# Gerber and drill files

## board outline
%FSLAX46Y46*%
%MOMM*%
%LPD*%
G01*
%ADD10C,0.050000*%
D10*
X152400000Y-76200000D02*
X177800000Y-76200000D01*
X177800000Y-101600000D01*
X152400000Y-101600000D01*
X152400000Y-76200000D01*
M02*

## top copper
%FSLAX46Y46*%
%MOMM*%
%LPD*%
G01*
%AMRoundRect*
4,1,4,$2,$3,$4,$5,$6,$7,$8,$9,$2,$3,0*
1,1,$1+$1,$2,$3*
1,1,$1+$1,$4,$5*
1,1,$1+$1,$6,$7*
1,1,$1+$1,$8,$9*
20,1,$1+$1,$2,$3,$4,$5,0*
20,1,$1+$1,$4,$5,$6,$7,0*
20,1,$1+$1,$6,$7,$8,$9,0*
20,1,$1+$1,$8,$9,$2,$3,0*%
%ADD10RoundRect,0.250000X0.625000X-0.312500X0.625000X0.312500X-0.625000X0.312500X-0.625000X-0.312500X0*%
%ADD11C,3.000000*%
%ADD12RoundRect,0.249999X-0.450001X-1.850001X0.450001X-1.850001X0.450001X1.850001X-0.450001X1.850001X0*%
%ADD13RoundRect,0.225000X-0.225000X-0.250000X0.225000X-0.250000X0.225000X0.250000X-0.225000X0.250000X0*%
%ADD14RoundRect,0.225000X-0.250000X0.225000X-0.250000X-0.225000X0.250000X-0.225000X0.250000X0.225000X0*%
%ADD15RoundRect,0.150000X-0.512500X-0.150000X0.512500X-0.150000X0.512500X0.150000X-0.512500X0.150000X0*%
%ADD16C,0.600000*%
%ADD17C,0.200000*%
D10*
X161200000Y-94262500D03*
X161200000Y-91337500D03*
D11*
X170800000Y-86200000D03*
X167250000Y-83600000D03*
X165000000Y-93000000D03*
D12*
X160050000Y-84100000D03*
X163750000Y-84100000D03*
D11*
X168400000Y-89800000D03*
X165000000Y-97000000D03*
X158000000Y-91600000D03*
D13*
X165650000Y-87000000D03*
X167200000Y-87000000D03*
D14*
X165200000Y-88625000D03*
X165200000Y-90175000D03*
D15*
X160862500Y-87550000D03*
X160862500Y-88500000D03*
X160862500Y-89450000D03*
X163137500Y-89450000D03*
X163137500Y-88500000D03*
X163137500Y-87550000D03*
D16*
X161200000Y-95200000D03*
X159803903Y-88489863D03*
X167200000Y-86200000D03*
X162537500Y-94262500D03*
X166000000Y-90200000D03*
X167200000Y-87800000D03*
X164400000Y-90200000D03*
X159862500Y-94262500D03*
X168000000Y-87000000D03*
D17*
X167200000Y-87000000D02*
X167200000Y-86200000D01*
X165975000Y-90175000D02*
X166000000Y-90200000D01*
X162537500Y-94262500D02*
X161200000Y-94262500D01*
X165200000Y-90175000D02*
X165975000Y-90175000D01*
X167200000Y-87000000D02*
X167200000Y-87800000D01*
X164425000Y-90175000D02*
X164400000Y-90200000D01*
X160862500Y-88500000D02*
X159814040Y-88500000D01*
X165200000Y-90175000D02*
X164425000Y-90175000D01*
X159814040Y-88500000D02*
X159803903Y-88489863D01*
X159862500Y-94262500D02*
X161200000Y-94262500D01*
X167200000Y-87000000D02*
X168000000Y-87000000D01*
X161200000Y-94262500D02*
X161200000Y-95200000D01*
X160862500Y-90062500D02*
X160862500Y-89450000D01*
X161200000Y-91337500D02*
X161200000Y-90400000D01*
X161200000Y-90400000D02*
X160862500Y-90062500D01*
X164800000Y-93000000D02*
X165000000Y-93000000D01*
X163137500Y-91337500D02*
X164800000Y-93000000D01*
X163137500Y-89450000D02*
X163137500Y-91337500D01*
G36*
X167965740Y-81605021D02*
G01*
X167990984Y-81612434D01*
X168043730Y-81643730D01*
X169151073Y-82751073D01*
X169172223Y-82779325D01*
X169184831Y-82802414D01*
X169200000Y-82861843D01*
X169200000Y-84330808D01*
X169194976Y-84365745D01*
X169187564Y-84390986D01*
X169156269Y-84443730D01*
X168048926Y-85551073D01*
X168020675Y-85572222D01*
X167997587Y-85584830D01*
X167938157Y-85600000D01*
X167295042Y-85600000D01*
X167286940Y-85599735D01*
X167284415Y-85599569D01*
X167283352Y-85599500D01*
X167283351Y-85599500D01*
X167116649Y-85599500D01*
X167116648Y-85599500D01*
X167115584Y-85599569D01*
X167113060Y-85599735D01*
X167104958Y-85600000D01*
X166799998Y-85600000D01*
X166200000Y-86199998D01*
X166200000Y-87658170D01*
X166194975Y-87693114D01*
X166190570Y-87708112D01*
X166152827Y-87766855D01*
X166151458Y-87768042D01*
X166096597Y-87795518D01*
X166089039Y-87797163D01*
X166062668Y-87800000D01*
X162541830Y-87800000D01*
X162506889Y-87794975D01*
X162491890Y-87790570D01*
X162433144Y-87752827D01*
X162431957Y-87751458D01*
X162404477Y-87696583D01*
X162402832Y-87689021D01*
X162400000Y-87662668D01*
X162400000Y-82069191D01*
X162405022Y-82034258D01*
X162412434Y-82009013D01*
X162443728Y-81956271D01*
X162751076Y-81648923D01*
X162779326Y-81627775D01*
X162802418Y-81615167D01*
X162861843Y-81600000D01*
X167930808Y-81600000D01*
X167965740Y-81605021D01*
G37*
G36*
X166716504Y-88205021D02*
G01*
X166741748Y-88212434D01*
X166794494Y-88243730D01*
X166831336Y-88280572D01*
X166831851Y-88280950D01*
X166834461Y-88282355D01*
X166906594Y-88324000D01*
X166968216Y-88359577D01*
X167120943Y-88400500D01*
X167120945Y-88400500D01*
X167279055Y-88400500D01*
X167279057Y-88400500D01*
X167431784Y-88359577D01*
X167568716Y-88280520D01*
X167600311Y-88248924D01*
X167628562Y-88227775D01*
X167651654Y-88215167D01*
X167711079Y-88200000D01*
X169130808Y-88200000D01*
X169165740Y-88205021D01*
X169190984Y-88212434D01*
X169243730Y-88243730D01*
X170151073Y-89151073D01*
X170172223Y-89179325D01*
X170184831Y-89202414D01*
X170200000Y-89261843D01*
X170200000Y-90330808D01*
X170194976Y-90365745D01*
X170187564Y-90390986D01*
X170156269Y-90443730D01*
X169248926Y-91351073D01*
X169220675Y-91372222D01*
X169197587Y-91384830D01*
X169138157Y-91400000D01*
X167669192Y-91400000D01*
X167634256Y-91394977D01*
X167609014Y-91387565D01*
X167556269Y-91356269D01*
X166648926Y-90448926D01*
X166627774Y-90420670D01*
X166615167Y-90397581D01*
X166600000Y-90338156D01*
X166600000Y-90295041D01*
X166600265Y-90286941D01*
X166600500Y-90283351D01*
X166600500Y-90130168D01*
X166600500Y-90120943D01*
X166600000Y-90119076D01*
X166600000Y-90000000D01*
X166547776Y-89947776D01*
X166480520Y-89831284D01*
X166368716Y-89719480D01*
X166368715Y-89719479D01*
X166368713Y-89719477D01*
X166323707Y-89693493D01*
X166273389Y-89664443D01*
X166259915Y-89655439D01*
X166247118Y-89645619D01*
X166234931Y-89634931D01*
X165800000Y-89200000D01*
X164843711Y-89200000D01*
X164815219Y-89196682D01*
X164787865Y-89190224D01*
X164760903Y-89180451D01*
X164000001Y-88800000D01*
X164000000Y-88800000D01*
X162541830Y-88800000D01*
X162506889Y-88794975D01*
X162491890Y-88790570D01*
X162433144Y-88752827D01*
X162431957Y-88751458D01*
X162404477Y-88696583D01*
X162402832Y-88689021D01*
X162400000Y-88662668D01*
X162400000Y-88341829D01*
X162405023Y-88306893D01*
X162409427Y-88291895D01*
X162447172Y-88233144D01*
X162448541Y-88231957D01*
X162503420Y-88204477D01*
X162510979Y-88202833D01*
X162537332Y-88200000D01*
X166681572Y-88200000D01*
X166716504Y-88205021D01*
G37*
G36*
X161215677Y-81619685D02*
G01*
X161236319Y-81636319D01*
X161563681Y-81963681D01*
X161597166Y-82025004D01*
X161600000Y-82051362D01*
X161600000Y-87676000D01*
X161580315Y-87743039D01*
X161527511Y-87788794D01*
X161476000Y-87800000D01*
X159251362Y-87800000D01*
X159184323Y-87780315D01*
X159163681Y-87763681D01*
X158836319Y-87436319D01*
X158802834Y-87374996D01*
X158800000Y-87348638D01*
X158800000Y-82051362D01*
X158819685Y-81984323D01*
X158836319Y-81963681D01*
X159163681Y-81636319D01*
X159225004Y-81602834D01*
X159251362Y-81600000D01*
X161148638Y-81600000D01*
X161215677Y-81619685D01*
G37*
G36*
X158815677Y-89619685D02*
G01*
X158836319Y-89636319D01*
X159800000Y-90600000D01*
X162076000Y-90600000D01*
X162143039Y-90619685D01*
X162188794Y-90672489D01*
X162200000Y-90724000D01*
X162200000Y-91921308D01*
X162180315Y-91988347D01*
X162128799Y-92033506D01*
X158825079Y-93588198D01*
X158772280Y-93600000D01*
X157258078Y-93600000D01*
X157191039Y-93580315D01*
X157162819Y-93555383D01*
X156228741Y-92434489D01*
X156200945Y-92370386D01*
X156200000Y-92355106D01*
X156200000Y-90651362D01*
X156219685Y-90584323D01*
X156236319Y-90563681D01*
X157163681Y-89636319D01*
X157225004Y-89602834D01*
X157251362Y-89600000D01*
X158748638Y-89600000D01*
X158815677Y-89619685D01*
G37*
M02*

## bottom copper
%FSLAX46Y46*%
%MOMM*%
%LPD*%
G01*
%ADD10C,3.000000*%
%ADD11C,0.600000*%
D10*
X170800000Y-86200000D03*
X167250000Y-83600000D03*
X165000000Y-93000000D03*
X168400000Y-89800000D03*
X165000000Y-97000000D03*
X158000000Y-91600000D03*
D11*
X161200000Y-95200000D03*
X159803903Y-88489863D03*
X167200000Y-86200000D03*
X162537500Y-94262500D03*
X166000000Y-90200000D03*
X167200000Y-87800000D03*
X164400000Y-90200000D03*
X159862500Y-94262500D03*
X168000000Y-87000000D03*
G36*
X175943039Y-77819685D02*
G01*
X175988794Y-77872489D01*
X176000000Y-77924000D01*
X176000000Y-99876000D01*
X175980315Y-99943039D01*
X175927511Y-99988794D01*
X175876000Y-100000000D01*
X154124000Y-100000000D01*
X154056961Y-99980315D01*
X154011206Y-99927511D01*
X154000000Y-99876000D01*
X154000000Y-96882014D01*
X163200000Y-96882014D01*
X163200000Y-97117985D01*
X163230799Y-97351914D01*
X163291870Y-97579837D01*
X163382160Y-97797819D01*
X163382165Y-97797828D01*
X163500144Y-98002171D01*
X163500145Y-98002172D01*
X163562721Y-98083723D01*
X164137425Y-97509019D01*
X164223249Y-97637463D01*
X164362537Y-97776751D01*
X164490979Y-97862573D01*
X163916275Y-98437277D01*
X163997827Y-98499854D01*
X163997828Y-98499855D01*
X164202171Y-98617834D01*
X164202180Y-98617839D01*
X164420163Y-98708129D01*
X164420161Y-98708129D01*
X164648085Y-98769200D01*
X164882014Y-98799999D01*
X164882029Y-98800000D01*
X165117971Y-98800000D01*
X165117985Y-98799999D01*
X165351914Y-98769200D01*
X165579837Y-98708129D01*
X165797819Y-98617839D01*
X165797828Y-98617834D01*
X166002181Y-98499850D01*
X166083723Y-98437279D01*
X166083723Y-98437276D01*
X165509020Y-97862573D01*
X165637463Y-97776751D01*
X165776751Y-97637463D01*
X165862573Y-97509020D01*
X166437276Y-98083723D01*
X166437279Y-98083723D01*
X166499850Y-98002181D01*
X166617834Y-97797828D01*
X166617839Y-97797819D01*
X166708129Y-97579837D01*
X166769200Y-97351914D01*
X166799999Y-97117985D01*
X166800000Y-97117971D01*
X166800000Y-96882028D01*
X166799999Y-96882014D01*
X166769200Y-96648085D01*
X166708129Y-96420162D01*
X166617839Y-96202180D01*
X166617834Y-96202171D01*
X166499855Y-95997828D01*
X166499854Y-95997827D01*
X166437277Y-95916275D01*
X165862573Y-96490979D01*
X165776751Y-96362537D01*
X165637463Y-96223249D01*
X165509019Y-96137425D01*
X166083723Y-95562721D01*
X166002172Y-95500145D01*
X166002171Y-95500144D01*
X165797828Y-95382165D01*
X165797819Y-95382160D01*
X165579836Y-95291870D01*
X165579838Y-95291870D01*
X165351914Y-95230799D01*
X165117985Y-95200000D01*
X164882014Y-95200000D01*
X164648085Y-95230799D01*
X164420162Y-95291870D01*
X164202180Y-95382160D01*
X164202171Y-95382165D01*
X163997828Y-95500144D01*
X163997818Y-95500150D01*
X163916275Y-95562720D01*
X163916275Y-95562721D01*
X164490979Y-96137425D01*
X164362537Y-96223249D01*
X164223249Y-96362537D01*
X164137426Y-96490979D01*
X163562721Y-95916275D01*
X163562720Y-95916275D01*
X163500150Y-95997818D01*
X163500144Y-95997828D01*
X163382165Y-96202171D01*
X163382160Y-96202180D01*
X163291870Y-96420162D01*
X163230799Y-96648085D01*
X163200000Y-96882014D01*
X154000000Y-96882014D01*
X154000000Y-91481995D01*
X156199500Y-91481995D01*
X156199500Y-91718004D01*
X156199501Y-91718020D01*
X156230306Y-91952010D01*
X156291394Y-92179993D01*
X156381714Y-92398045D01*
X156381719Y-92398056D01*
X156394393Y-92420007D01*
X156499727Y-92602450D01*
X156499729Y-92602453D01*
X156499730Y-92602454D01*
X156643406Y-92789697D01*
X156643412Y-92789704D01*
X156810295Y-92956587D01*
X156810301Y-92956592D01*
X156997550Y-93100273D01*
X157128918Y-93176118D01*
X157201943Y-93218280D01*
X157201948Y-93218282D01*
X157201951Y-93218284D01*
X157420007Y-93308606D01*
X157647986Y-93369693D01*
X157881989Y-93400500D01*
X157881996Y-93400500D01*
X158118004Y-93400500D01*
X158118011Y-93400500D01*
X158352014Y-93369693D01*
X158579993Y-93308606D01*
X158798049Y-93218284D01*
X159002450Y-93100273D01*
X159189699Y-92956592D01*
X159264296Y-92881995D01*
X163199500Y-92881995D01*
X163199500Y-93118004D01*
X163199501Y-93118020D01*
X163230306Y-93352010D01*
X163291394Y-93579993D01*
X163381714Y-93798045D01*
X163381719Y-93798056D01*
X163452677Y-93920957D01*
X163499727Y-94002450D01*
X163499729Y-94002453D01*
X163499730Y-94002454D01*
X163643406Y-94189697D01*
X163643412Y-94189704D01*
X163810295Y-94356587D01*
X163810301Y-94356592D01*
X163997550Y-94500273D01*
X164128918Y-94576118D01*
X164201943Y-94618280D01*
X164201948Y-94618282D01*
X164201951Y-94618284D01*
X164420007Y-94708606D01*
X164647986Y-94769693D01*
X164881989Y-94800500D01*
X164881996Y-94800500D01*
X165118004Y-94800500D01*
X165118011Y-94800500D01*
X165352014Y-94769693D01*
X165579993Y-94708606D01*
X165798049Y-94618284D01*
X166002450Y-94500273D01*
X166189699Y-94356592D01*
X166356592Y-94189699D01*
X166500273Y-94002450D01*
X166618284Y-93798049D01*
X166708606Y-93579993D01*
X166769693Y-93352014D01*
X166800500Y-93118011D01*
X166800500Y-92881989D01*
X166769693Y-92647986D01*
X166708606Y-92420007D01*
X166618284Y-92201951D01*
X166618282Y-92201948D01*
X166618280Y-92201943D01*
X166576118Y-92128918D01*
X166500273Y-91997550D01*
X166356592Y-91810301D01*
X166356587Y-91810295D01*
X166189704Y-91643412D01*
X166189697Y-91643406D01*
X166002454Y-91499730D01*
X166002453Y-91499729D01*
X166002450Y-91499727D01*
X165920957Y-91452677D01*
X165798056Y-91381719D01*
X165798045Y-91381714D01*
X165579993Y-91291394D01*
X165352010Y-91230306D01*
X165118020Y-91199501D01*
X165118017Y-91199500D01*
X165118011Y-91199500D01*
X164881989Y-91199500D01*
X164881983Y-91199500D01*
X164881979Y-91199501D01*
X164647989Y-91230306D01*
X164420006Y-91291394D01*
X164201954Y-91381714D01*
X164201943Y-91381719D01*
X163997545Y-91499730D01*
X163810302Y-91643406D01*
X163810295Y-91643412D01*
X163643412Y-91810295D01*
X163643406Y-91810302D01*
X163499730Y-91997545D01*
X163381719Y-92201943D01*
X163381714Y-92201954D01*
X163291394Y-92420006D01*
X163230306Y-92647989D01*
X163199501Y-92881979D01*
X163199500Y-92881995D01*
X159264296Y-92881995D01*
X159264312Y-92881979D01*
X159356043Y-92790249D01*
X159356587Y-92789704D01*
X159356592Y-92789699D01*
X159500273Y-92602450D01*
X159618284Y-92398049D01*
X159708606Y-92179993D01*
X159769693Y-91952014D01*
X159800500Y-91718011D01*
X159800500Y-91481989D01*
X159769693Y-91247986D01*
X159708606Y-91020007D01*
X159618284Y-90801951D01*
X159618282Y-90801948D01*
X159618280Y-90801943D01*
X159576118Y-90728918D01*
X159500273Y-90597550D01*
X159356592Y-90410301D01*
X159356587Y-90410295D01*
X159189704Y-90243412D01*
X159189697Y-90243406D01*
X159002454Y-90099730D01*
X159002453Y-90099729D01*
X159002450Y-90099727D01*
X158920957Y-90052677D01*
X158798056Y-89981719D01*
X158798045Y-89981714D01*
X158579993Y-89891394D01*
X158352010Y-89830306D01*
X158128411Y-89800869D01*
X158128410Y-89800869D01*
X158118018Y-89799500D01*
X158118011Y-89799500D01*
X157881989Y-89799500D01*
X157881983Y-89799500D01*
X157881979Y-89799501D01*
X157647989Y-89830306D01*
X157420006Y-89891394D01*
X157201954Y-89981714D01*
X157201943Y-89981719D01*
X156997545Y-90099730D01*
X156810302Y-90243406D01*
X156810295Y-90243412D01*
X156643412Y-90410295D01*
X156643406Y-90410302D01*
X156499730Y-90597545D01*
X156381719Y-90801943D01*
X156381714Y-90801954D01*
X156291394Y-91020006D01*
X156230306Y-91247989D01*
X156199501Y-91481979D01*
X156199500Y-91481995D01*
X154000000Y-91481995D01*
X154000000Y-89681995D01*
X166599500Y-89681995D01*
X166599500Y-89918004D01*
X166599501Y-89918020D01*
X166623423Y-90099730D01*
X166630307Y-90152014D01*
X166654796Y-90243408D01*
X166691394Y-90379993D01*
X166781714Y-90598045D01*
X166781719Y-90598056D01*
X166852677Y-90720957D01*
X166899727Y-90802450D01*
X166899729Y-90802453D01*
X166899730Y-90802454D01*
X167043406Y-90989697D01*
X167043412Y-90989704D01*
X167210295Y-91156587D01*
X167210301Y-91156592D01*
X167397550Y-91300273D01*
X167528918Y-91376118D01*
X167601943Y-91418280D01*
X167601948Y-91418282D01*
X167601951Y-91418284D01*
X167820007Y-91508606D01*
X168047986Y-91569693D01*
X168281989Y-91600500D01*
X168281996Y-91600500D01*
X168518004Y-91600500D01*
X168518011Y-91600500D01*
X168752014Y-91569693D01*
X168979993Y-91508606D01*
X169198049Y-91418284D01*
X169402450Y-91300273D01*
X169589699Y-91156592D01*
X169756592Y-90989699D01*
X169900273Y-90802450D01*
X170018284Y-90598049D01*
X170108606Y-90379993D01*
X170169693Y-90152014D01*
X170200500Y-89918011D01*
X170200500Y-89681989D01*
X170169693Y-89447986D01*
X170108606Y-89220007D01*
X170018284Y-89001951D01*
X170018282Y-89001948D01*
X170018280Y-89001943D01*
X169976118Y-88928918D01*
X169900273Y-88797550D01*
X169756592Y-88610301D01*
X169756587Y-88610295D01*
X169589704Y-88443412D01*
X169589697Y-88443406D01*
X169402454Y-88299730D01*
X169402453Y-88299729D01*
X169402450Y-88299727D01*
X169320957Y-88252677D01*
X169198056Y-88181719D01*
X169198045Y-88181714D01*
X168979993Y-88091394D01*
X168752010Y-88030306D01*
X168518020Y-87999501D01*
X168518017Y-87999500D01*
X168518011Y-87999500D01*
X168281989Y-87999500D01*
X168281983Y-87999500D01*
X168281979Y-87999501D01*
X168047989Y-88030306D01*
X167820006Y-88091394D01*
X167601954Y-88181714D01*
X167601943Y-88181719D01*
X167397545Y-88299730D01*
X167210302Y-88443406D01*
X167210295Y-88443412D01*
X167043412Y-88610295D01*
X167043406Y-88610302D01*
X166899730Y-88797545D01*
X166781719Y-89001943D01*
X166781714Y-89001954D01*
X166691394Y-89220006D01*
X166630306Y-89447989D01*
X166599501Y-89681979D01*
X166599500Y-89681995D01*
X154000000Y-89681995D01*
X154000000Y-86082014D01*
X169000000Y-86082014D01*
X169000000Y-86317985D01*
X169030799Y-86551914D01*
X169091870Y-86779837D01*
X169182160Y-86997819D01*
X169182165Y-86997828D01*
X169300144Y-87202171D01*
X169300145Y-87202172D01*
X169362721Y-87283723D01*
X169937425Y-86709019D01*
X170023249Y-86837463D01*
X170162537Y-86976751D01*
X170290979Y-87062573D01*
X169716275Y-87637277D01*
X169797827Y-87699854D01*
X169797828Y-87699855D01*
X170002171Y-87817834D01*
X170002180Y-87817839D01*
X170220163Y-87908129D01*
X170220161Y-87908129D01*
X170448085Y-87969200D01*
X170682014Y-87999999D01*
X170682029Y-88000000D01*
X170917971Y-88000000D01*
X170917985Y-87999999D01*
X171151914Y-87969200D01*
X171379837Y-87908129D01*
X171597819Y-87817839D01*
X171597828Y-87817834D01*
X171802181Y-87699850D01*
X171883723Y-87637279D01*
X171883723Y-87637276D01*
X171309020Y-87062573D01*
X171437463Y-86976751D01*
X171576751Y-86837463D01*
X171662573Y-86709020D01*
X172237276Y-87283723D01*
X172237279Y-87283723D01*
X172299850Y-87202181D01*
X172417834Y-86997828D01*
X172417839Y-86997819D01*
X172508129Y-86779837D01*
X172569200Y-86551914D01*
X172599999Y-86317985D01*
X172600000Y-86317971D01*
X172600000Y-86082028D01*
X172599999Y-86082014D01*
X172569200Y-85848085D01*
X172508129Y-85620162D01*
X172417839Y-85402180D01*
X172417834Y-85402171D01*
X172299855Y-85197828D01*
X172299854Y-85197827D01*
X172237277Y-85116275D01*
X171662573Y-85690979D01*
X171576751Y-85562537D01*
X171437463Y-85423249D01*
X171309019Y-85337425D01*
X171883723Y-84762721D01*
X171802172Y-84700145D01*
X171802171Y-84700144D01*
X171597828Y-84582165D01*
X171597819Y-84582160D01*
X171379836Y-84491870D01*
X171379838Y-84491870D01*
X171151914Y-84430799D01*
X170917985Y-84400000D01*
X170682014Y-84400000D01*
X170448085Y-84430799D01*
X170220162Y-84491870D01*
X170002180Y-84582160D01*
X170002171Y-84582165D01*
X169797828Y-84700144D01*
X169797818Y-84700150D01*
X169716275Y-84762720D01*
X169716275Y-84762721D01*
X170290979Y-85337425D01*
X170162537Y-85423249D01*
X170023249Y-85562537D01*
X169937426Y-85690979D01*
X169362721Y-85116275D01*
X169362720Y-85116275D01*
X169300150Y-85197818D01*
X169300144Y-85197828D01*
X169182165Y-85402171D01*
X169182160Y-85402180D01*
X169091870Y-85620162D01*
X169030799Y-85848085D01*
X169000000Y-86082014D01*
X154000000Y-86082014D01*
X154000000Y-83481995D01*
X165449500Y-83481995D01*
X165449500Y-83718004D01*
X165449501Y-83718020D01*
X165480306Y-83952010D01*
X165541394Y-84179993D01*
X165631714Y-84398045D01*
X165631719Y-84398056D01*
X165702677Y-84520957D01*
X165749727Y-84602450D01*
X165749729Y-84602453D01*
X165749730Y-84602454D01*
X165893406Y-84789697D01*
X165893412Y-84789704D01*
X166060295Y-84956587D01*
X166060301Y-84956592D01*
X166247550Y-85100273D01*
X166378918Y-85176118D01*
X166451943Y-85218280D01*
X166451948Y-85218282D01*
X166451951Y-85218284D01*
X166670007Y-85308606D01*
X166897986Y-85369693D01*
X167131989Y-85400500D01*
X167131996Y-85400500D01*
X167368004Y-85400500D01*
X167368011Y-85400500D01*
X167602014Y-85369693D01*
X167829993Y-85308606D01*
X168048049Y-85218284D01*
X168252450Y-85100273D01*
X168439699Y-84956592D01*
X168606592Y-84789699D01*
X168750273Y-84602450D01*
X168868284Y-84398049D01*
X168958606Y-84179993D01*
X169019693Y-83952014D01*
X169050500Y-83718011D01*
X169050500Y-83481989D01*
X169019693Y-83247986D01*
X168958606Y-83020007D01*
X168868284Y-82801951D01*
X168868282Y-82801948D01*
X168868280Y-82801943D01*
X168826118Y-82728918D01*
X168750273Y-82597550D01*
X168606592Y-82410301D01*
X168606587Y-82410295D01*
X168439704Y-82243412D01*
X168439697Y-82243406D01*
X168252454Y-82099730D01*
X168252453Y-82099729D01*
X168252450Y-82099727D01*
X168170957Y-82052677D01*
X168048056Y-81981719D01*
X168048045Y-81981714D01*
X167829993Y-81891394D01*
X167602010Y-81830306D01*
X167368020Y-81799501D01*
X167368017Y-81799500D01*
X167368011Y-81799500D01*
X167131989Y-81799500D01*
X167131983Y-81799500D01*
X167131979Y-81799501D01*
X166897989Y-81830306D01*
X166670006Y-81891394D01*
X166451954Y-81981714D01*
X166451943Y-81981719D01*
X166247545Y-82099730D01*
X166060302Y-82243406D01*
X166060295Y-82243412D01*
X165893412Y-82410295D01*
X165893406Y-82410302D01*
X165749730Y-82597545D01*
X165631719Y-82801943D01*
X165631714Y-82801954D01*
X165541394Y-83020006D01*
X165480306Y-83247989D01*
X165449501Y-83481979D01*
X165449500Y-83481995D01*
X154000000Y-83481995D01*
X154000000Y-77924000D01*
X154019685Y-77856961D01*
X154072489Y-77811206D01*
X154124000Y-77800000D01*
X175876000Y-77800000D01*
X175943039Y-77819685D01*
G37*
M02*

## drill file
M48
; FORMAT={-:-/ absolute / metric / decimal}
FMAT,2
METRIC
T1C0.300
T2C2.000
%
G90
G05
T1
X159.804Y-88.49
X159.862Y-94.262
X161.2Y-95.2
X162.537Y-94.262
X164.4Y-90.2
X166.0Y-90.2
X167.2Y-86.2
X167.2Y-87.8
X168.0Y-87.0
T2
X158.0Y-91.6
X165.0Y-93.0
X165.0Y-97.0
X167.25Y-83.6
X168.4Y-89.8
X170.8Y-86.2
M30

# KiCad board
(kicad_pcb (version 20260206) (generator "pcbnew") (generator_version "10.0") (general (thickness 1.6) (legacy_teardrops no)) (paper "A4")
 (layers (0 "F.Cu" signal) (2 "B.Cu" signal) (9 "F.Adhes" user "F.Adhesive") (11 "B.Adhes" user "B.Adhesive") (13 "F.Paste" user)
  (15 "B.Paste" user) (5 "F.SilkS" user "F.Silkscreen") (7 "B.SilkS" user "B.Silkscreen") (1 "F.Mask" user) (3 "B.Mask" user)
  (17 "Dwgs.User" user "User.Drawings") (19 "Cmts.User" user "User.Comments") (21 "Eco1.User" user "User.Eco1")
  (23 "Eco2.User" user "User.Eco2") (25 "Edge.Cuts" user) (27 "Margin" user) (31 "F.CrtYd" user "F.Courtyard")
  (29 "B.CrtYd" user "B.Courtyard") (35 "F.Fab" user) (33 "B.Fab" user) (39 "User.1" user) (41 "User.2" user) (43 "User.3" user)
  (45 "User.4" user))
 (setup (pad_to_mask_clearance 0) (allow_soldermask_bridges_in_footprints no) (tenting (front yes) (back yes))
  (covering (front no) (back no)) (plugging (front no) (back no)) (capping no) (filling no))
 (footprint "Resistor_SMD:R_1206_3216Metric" (layer "F.Cu") (at 161.2 92.8 90)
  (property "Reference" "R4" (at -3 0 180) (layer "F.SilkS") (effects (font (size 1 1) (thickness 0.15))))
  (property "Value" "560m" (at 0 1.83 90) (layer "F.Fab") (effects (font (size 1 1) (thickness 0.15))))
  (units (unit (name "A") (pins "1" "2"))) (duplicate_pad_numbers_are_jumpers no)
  (pad "1" smd roundrect (at -1.4625 0 90) (size 1.125 1.75) (layers "F.Cu" "F.Mask" "F.Paste") (roundrect_rratio 0.222222) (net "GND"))
  (pad "2" smd roundrect (at 1.4625 0 90) (size 1.125 1.75) (layers "F.Cu" "F.Mask" "F.Paste") (roundrect_rratio 0.222222)
   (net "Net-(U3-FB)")))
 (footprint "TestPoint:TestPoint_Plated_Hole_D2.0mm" (layer "F.Cu") (at 170.8 86.2 90)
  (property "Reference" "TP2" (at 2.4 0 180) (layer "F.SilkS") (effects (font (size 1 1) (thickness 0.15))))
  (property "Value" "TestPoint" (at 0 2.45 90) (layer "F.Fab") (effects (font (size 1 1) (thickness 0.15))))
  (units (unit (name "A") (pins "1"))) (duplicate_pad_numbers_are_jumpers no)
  (pad "1" thru_hole circle (at 0 0 90) (size 3 3) (drill 2) (layers "*.Cu" "*.Mask") (remove_unused_layers no) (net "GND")))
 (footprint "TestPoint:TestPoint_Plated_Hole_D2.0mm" (layer "F.Cu") (at 167.25 83.6 90)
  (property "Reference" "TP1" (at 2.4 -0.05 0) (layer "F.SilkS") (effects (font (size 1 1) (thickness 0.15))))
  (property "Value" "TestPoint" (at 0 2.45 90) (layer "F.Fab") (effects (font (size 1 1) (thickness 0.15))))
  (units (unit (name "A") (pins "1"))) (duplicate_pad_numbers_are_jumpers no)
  (pad "1" thru_hole circle (at 0 0 90) (size 3 3) (drill 2) (layers "*.Cu" "*.Mask") (remove_unused_layers no) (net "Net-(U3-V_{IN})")))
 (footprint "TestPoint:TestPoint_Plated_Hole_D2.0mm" (layer "F.Cu") (at 165 93 90)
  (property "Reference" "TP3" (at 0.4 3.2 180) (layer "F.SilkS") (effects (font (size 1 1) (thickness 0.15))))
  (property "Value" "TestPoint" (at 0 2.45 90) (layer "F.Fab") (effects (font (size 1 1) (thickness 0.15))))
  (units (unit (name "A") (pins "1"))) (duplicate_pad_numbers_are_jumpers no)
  (pad "1" thru_hole circle (at 0 0 90) (size 3 3) (drill 2) (layers "*.Cu" "*.Mask") (remove_unused_layers no) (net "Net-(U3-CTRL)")))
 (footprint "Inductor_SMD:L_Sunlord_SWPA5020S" (layer "F.Cu") (at 161.9 84.1)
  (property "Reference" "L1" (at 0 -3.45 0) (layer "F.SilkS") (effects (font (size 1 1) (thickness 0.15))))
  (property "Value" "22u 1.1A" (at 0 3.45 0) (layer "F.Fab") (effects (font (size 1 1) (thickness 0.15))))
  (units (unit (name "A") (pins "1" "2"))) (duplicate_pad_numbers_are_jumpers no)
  (pad "1" smd roundrect (at -1.85 0) (size 1.4 4.2) (layers "F.Cu" "F.Mask" "F.Paste") (roundrect_rratio 0.178571) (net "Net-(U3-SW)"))
  (pad "2" smd roundrect (at 1.85 0) (size 1.4 4.2) (layers "F.Cu" "F.Mask" "F.Paste") (roundrect_rratio 0.178571) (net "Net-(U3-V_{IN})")))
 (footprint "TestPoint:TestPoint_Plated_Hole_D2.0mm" (layer "F.Cu") (at 168.4 89.8 90)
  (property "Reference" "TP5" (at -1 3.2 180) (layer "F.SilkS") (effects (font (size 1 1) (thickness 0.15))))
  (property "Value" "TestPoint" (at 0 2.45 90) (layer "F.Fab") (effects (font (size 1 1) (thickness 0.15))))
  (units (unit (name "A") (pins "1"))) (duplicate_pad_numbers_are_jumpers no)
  (pad "1" thru_hole circle (at 0 0 90) (size 3 3) (drill 2) (layers "*.Cu" "*.Mask") (remove_unused_layers no) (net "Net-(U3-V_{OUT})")))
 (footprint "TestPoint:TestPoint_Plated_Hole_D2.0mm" (layer "F.Cu") (at 165 97 90)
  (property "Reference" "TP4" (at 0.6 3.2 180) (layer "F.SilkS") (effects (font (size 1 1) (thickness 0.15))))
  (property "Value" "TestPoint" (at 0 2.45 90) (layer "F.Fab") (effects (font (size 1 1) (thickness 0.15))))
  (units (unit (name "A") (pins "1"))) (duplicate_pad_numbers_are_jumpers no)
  (pad "1" thru_hole circle (at 0 0 90) (size 3 3) (drill 2) (layers "*.Cu" "*.Mask") (remove_unused_layers no) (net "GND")))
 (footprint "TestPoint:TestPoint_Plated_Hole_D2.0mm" (layer "F.Cu") (at 158 91.6 90)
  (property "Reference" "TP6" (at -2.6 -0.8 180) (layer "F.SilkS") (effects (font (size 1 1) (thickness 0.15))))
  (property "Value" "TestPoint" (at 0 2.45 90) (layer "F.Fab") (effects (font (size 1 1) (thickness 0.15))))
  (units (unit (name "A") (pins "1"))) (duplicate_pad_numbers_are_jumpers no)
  (pad "1" thru_hole circle (at 0 0 90) (size 3 3) (drill 2) (layers "*.Cu" "*.Mask") (remove_unused_layers no) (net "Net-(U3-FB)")))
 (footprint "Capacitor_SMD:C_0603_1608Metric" (layer "F.Cu") (at 166.425 87)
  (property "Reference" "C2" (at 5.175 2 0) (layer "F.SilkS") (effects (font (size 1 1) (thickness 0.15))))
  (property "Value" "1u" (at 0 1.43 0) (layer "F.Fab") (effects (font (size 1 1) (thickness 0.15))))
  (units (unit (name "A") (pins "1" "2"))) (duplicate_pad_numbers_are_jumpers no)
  (pad "1" smd roundrect (at -0.775 0) (size 0.9 0.95) (layers "F.Cu" "F.Mask" "F.Paste") (roundrect_rratio 0.25) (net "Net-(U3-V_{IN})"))
  (pad "2" smd roundrect (at 0.775 0) (size 0.9 0.95) (layers "F.Cu" "F.Mask" "F.Paste") (roundrect_rratio 0.25) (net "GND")))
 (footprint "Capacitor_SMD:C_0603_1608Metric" (layer "F.Cu") (at 165.2 89.4 -90)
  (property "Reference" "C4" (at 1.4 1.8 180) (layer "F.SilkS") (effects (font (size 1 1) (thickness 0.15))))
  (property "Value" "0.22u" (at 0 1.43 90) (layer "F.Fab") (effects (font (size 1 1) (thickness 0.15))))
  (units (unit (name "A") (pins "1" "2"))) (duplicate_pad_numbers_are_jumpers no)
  (pad "1" smd roundrect (at -0.775 0 270) (size 0.9 0.95) (layers "F.Cu" "F.Mask" "F.Paste") (roundrect_rratio 0.25)
   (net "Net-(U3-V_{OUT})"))
  (pad "2" smd roundrect (at 0.775 0 270) (size 0.9 0.95) (layers "F.Cu" "F.Mask" "F.Paste") (roundrect_rratio 0.25) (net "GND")))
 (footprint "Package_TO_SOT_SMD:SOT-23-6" (layer "F.Cu") (at 162 88.5)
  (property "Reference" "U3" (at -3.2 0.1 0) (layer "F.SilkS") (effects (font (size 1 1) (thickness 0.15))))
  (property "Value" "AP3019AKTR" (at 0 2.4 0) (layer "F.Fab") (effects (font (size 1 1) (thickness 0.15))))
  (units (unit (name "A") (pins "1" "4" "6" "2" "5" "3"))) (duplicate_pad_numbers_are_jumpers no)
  (pad "1" smd roundrect (at -1.1375 -0.95) (size 1.325 0.6) (layers "F.Cu" "F.Mask" "F.Paste") (roundrect_rratio 0.25) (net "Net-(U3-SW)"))
  (pad "2" smd roundrect (at -1.1375 0) (size 1.325 0.6) (layers "F.Cu" "F.Mask" "F.Paste") (roundrect_rratio 0.25) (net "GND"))
  (pad "3" smd roundrect (at -1.1375 0.95) (size 1.325 0.6) (layers "F.Cu" "F.Mask" "F.Paste") (roundrect_rratio 0.25) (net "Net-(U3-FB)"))
  (pad "4" smd roundrect (at 1.1375 0.95) (size 1.325 0.6) (layers "F.Cu" "F.Mask" "F.Paste") (roundrect_rratio 0.25) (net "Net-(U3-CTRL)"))
  (pad "5" smd roundrect (at 1.1375 0) (size 1.325 0.6) (layers "F.Cu" "F.Mask" "F.Paste") (roundrect_rratio 0.25) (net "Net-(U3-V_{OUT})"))
  (pad "6" smd roundrect (at 1.1375 -0.95) (size 1.325 0.6) (layers "F.Cu" "F.Mask" "F.Paste") (roundrect_rratio 0.25)
   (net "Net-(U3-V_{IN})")))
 (gr_rect (start 152.4 76.2) (end 177.8 101.6) (stroke (width 0.05) (type default)) (fill no) (layer "Edge.Cuts"))
 (segment (start 167.2 87) (end 167.2 86.2) (width 0.2) (layer "F.Cu") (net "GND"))
 (segment (start 165.975 90.175) (end 166 90.2) (width 0.2) (layer "F.Cu") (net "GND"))
 (segment (start 162.5375 94.2625) (end 161.2 94.2625) (width 0.2) (layer "F.Cu") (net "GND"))
 (segment (start 165.2 90.175) (end 165.975 90.175) (width 0.2) (layer "F.Cu") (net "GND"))
 (segment (start 167.2 87) (end 167.2 87.8) (width 0.2) (layer "F.Cu") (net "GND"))
 (segment (start 164.425 90.175) (end 164.4 90.2) (width 0.2) (layer "F.Cu") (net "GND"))
 (segment (start 160.8625 88.5) (end 159.81404 88.5) (width 0.2) (layer "F.Cu") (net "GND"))
 (segment (start 165.2 90.175) (end 164.425 90.175) (width 0.2) (layer "F.Cu") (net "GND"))
 (segment (start 159.81404 88.5) (end 159.803903 88.489863) (width 0.2) (layer "F.Cu") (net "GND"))
 (segment (start 159.8625 94.2625) (end 161.2 94.2625) (width 0.2) (layer "F.Cu") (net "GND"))
 (segment (start 167.2 87) (end 168 87) (width 0.2) (layer "F.Cu") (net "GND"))
 (segment (start 161.2 94.2625) (end 161.2 95.2) (width 0.2) (layer "F.Cu") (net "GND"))
 (via (at 161.2 95.2) (size 0.6) (drill 0.3) (layers "F.Cu" "B.Cu") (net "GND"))
 (via (at 159.803903 88.489863) (size 0.6) (drill 0.3) (layers "F.Cu" "B.Cu") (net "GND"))
 (via (at 167.2 86.2) (size 0.6) (drill 0.3) (layers "F.Cu" "B.Cu") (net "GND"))
 (via (at 162.5375 94.2625) (size 0.6) (drill 0.3) (layers "F.Cu" "B.Cu") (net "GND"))
 (via (at 166 90.2) (size 0.6) (drill 0.3) (layers "F.Cu" "B.Cu") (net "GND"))
 (via (at 167.2 87.8) (size 0.6) (drill 0.3) (layers "F.Cu" "B.Cu") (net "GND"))
 (via (at 164.4 90.2) (size 0.6) (drill 0.3) (layers "F.Cu" "B.Cu") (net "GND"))
 (via (at 159.8625 94.2625) (size 0.6) (drill 0.3) (layers "F.Cu" "B.Cu") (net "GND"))
 (via (at 168 87) (size 0.6) (drill 0.3) (layers "F.Cu" "B.Cu") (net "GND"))
 (segment (start 160.8625 90.0625) (end 160.8625 89.45) (width 0.2) (layer "F.Cu") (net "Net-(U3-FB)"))
 (segment (start 161.2 91.3375) (end 161.2 90.4) (width 0.2) (layer "F.Cu") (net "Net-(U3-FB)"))
 (segment (start 161.2 90.4) (end 160.8625 90.0625) (width 0.2) (layer "F.Cu") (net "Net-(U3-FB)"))
 (segment (start 164.8 93) (end 165 93) (width 0.2) (layer "F.Cu") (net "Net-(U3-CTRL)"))
 (segment (start 163.1375 91.3375) (end 164.8 93) (width 0.2) (layer "F.Cu") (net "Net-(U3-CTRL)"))
 (segment (start 163.1375 89.45) (end 163.1375 91.3375) (width 0.2) (layer "F.Cu") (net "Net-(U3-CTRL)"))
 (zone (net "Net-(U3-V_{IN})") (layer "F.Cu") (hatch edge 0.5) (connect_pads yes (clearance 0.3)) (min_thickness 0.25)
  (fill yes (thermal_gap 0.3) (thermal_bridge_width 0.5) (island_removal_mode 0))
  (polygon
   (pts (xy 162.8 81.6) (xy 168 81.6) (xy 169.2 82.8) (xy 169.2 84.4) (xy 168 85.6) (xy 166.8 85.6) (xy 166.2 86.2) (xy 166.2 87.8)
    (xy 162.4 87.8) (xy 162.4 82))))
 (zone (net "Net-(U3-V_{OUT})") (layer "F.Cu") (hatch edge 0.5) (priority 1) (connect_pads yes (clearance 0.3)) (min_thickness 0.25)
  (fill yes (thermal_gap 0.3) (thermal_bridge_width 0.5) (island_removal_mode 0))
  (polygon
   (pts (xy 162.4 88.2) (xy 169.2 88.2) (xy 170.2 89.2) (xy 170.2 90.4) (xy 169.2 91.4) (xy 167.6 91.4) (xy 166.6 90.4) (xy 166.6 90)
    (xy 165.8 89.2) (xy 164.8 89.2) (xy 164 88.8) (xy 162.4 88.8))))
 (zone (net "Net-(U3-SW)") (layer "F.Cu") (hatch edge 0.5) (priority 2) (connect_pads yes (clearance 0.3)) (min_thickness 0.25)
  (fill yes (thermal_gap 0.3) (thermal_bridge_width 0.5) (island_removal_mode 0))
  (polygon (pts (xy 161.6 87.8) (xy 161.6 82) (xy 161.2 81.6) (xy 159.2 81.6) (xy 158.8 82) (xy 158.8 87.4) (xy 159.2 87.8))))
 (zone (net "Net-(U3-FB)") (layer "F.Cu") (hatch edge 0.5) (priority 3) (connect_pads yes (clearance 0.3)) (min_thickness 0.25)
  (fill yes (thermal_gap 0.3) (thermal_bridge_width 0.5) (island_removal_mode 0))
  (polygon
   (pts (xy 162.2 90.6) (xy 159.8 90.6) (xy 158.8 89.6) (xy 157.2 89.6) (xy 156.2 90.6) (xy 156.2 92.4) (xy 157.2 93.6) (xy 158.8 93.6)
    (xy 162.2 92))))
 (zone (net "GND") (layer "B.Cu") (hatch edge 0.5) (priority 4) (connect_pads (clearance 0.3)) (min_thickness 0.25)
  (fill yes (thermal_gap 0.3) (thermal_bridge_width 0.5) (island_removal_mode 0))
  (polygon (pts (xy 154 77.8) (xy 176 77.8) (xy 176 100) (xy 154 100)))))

